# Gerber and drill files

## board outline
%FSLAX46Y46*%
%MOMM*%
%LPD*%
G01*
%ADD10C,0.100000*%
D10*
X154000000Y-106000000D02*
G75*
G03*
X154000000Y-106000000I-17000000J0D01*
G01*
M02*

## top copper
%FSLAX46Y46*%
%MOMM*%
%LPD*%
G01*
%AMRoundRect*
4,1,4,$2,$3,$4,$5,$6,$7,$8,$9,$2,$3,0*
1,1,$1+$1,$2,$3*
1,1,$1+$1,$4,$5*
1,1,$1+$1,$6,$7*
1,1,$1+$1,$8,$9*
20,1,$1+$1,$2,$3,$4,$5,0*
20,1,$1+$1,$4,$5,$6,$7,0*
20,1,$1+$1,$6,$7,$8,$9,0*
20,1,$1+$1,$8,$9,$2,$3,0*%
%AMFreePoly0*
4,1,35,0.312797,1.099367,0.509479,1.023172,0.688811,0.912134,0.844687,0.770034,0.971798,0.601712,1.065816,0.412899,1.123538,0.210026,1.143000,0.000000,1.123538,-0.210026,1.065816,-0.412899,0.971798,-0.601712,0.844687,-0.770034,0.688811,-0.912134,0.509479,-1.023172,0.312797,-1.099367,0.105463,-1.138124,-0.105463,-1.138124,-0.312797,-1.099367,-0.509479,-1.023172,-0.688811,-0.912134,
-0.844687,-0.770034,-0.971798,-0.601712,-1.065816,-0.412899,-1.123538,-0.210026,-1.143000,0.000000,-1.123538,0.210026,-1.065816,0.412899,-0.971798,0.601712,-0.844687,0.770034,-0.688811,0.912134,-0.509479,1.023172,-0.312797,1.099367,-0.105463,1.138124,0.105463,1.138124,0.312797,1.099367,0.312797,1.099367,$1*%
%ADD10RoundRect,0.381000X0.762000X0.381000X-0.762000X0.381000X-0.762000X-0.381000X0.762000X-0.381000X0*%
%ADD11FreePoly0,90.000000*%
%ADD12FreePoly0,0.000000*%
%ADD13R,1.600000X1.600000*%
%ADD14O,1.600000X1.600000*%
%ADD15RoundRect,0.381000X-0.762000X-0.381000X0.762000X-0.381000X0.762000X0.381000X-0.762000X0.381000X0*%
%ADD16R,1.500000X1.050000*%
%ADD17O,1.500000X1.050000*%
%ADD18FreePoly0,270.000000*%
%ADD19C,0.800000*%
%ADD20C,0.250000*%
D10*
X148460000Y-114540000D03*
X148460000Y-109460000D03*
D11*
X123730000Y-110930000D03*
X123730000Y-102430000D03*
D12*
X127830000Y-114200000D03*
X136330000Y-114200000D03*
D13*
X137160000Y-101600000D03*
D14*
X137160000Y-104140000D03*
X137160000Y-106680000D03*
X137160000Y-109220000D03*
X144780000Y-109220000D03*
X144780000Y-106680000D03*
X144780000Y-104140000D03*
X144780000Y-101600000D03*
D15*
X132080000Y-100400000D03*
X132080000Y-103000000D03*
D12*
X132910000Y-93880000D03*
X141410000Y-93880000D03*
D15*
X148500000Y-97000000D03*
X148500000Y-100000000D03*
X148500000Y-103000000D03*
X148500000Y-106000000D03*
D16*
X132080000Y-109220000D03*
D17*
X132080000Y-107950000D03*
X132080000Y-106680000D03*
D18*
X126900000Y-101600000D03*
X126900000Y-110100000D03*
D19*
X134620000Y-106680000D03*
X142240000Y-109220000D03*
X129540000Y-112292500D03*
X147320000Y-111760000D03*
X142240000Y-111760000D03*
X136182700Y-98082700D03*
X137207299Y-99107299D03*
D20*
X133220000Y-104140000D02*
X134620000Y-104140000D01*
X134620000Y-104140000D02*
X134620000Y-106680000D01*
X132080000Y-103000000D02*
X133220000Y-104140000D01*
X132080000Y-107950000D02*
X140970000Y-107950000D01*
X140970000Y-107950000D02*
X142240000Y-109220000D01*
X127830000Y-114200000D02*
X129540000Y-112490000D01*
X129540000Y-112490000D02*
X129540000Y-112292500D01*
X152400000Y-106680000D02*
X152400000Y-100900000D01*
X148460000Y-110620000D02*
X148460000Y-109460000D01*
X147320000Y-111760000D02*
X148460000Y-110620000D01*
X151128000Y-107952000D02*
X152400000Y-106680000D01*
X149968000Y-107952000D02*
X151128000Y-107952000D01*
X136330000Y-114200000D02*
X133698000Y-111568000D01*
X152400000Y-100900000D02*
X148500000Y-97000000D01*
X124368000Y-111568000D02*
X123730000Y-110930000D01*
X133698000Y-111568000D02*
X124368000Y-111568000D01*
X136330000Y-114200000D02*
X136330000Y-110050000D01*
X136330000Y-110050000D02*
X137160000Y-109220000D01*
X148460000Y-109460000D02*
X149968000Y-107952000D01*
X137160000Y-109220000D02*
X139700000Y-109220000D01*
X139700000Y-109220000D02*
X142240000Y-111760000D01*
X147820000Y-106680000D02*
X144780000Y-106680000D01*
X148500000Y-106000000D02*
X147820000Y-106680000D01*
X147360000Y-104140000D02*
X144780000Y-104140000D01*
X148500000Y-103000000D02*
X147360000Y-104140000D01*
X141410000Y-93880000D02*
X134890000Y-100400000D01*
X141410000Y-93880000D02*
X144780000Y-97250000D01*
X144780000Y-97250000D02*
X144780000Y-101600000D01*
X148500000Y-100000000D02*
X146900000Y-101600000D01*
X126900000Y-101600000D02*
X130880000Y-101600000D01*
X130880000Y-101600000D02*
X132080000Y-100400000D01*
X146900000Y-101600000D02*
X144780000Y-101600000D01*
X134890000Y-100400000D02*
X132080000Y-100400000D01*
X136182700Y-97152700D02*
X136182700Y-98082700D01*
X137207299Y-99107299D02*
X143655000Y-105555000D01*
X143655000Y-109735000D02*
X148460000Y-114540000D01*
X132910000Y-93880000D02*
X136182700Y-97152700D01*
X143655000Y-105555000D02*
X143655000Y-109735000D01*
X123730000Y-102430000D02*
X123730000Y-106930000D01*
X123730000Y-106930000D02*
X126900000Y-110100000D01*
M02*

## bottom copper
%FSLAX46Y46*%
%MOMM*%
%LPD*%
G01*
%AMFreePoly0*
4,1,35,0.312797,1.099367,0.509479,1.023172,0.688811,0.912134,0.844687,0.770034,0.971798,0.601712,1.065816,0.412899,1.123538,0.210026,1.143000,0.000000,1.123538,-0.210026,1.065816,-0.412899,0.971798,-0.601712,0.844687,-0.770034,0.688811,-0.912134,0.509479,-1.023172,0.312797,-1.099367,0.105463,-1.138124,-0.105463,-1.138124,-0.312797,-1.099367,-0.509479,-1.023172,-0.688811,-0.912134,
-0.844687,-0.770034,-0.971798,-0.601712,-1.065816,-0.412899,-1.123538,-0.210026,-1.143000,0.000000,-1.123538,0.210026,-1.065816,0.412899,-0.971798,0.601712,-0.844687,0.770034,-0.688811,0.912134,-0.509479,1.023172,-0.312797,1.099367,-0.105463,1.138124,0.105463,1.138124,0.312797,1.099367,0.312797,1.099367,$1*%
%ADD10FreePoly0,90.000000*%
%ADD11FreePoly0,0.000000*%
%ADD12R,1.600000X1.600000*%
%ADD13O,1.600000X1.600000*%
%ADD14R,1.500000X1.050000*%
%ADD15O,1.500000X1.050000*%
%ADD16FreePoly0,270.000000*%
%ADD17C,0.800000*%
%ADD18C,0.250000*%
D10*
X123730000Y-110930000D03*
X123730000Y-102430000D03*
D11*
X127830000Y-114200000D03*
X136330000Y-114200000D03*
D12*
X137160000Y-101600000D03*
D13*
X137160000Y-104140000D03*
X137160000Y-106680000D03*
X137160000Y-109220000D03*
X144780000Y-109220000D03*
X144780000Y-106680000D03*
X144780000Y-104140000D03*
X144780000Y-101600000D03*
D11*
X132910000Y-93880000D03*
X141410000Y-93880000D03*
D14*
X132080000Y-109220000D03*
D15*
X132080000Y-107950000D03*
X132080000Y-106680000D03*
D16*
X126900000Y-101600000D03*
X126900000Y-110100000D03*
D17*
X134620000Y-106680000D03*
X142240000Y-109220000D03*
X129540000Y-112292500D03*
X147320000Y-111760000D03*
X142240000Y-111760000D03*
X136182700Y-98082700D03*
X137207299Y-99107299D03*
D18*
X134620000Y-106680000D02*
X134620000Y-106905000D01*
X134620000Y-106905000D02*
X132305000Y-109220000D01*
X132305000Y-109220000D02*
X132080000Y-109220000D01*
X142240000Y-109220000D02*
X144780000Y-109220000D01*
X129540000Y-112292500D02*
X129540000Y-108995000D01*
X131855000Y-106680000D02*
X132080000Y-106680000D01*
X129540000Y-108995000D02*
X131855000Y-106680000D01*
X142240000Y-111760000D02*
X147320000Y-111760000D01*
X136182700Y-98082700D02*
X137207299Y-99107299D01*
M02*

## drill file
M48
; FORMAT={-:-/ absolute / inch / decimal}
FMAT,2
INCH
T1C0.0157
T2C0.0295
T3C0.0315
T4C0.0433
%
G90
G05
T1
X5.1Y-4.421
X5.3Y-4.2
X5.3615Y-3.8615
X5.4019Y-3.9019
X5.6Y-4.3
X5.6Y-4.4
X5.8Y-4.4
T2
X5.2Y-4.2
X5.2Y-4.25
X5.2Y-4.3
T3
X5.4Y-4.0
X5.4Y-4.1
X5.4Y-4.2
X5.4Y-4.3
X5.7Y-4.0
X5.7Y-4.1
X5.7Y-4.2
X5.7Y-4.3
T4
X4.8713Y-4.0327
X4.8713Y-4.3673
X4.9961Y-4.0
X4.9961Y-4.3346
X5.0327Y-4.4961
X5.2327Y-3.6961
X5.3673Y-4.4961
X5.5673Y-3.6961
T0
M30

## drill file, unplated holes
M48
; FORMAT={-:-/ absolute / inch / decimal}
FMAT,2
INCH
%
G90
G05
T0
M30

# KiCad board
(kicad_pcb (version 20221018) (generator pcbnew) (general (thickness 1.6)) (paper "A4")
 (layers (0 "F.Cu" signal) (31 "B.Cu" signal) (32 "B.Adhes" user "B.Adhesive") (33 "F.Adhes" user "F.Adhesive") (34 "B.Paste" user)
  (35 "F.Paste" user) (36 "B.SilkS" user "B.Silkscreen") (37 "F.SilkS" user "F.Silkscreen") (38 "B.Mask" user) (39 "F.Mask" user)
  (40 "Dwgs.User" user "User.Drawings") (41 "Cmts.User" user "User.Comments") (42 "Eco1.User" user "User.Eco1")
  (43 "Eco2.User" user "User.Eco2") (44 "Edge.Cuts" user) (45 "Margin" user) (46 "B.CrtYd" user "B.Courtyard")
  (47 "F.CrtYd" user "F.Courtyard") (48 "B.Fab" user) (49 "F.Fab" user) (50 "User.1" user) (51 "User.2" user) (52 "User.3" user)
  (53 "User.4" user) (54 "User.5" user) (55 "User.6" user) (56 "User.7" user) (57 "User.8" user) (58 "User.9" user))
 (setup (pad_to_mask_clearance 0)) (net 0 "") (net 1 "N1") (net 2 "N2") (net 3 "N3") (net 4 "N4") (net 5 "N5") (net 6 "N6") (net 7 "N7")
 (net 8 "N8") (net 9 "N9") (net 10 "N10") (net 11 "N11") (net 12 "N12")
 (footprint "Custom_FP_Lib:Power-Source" (layer "F.Cu") (at 151 112 180)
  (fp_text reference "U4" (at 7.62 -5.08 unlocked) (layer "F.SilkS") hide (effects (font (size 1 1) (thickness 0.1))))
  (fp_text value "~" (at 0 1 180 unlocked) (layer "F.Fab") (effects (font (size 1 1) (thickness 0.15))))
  (pad "1" smd roundrect (at 2.54 -2.54 180) (size 2.286 1.524) (layers "F.Cu" "F.Paste" "F.Mask") (roundrect_rratio 0.25) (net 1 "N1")
   (thermal_bridge_angle 45))
  (pad "2" smd roundrect (at 2.54 2.54 180) (size 2.286 1.524) (layers "F.Cu" "F.Paste" "F.Mask") (roundrect_rratio 0.25) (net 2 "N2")
   (thermal_bridge_angle 45)))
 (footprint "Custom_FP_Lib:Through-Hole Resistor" (layer "F.Cu") (at 125 111.25 90)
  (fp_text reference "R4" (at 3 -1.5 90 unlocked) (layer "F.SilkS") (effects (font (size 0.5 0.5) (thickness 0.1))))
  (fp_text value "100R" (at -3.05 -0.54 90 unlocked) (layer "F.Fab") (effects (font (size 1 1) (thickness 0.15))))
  (pad "1" thru_hole custom (at 0.32 -1.27 90) (size 2.286 2.286) (drill 1.1) (layers "*.Cu" "*.Mask") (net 2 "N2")
   (thermal_bridge_angle 45) (options (clearance outline) (anchor circle)) (primitives))
  (pad "2" thru_hole custom (at 8.82 -1.27 90) (size 2.286 2.286) (drill 1.1) (layers "*.Cu" "*.Mask") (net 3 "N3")
   (thermal_bridge_angle 45) (options (clearance outline) (anchor circle)) (primitives)))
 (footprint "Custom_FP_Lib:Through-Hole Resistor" (layer "F.Cu") (at 127.51 115.47)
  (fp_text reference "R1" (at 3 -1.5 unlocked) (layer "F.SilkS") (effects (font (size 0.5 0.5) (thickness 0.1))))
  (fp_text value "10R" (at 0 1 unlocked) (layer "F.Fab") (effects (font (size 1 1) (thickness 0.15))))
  (pad "1" thru_hole custom (at 0.32 -1.27) (size 2.286 2.286) (drill 1.1) (layers "*.Cu" "*.Mask") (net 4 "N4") (thermal_bridge_angle 45)
   (options (clearance outline) (anchor circle)) (primitives))
  (pad "2" thru_hole custom (at 8.82 -1.27) (size 2.286 2.286) (drill 1.1) (layers "*.Cu" "*.Mask") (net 2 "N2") (thermal_bridge_angle 45)
   (options (clearance outline) (anchor circle)) (primitives)))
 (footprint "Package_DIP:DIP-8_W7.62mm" (layer "F.Cu") (at 137.16 101.6)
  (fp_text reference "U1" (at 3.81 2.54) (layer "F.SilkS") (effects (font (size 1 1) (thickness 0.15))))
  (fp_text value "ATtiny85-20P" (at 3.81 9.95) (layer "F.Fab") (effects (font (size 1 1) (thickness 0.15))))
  (pad "1" thru_hole rect (at 0 0) (size 1.6 1.6) (drill 0.8) (layers "*.Cu" "*.Mask") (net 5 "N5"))
  (pad "2" thru_hole oval (at 0 2.54) (size 1.6 1.6) (drill 0.8) (layers "*.Cu" "*.Mask") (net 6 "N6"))
  (pad "3" thru_hole oval (at 0 5.08) (size 1.6 1.6) (drill 0.8) (layers "*.Cu" "*.Mask") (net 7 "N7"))
  (pad "4" thru_hole oval (at 0 7.62) (size 1.6 1.6) (drill 0.8) (layers "*.Cu" "*.Mask") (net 2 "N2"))
  (pad "5" thru_hole oval (at 7.62 7.62) (size 1.6 1.6) (drill 0.8) (layers "*.Cu" "*.Mask") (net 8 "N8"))
  (pad "6" thru_hole oval (at 7.62 5.08) (size 1.6 1.6) (drill 0.8) (layers "*.Cu" "*.Mask") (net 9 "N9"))
  (pad "7" thru_hole oval (at 7.62 2.54) (size 1.6 1.6) (drill 0.8) (layers "*.Cu" "*.Mask") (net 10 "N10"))
  (pad "8" thru_hole oval (at 7.62 0) (size 1.6 1.6) (drill 0.8) (layers "*.Cu" "*.Mask") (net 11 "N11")))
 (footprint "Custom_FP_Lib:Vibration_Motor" (layer "F.Cu") (at 132.08 103)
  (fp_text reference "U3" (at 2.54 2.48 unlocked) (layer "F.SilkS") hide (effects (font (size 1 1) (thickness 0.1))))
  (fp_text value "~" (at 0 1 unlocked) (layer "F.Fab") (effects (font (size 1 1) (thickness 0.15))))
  (pad "1" smd roundrect (at 0 -2.6) (size 2.286 1.524) (layers "F.Cu" "F.Paste" "F.Mask") (roundrect_rratio 0.25) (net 11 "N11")
   (thermal_bridge_angle 45))
  (pad "2" smd roundrect (at 0 0) (size 2.286 1.524) (layers "F.Cu" "F.Paste" "F.Mask") (roundrect_rratio 0.25) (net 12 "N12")
   (thermal_bridge_angle 45)))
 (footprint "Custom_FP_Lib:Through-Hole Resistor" (layer "F.Cu") (at 132.59 95.15)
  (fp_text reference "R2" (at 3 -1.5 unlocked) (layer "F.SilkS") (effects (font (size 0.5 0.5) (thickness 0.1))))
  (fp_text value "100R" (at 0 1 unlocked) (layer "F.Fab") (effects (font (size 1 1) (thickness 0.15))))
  (pad "1" thru_hole custom (at 0.32 -1.27) (size 2.286 2.286) (drill 1.1) (layers "*.Cu" "*.Mask") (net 1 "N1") (thermal_bridge_angle 45)
   (options (clearance outline) (anchor circle)) (primitives))
  (pad "2" thru_hole custom (at 8.82 -1.27) (size 2.286 2.286) (drill 1.1) (layers "*.Cu" "*.Mask") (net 11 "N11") (thermal_bridge_angle 45)
   (options (clearance outline) (anchor circle)) (primitives)))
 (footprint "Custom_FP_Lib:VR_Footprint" (layer "F.Cu") (at 148.5 103)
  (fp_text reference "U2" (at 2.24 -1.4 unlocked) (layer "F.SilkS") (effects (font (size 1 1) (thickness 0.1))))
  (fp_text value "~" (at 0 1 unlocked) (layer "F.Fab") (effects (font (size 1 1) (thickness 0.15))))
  (pad "1" smd roundrect (at 0 -6) (size 2.286 1.524) (layers "F.Cu" "F.Paste" "F.Mask") (roundrect_rratio 0.25) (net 2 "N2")
   (thermal_bridge_angle 45))
  (pad "2" smd roundrect (at 0 -3) (size 2.286 1.524) (layers "F.Cu" "F.Paste" "F.Mask") (roundrect_rratio 0.25) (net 11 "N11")
   (thermal_bridge_angle 45))
  (pad "3" smd roundrect (at 0 0) (size 2.286 1.524) (layers "F.Cu" "F.Paste" "F.Mask") (roundrect_rratio 0.25) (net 10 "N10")
   (thermal_bridge_angle 45))
  (pad "4" smd roundrect (at 0 3) (size 2.286 1.524) (layers "F.Cu" "F.Paste" "F.Mask") (roundrect_rratio 0.25) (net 9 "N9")
   (thermal_bridge_angle 45)))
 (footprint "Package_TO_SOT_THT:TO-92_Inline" (layer "F.Cu") (at 132.08 109.22 90)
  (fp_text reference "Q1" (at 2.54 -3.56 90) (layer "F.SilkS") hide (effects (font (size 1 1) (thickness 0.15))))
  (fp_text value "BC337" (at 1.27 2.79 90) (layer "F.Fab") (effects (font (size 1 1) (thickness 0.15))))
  (pad "1" thru_hole rect (at 0 0 90) (size 1.05 1.5) (drill 0.75) (layers "*.Cu" "*.Mask") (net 12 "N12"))
  (pad "2" thru_hole oval (at 1.27 0 90) (size 1.05 1.5) (drill 0.75) (layers "*.Cu" "*.Mask") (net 8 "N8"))
  (pad "3" thru_hole oval (at 2.54 0 90) (size 1.05 1.5) (drill 0.75) (layers "*.Cu" "*.Mask") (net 4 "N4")))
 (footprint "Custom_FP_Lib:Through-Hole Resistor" (layer "F.Cu") (at 125.63 101.28 -90)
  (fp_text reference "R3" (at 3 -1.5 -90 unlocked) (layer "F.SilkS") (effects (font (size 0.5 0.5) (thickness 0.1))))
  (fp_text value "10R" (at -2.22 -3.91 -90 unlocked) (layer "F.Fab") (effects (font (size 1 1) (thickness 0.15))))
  (pad "1" thru_hole custom (at 0.32 -1.27 270) (size 2.286 2.286) (drill 1.1) (layers "*.Cu" "*.Mask") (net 11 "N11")
   (thermal_bridge_angle 45) (options (clearance outline) (anchor circle)) (primitives))
  (pad "2" thru_hole custom (at 8.82 -1.27 270) (size 2.286 2.286) (drill 1.1) (layers "*.Cu" "*.Mask") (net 3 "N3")
   (thermal_bridge_angle 45) (options (clearance outline) (anchor circle)) (primitives)))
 (gr_circle (center 137 106) (end 154 106) (stroke (width 0.1) (type default)) (fill none) (layer "Edge.Cuts"))
 (segment (start 133.22 104.14) (end 134.62 104.14) (width 0.25) (layer "F.Cu") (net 12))
 (segment (start 134.62 104.14) (end 134.62 106.68) (width 0.25) (layer "F.Cu") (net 12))
 (segment (start 132.08 103) (end 133.22 104.14) (width 0.25) (layer "F.Cu") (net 12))
 (via (at 134.62 106.68) (size 0.8) (drill 0.4) (layers "F.Cu" "B.Cu") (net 12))
 (segment (start 134.62 106.68) (end 134.62 106.905) (width 0.25) (layer "B.Cu") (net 12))
 (segment (start 134.62 106.905) (end 132.305 109.22) (width 0.25) (layer "B.Cu") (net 12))
 (segment (start 132.305 109.22) (end 132.08 109.22) (width 0.25) (layer "B.Cu") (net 12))
 (segment (start 132.08 107.95) (end 140.97 107.95) (width 0.25) (layer "F.Cu") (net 8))
 (segment (start 140.97 107.95) (end 142.24 109.22) (width 0.25) (layer "F.Cu") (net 8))
 (via (at 142.24 109.22) (size 0.8) (drill 0.4) (layers "F.Cu" "B.Cu") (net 8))
 (segment (start 142.24 109.22) (end 144.78 109.22) (width 0.25) (layer "B.Cu") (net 8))
 (segment (start 127.83 114.2) (end 129.54 112.49) (width 0.25) (layer "F.Cu") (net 4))
 (segment (start 129.54 112.49) (end 129.54 112.2925) (width 0.25) (layer "F.Cu") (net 4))
 (via (at 129.54 112.2925) (size 0.8) (drill 0.4) (layers "F.Cu" "B.Cu") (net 4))
 (segment (start 129.54 112.2925) (end 129.54 108.995) (width 0.25) (layer "B.Cu") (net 4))
 (segment (start 131.855 106.68) (end 132.08 106.68) (width 0.25) (layer "B.Cu") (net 4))
 (segment (start 129.54 108.995) (end 131.855 106.68) (width 0.25) (layer "B.Cu") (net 4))
 (segment (start 152.4 106.68) (end 152.4 100.9) (width 0.25) (layer "F.Cu") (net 2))
 (segment (start 148.46 110.62) (end 148.46 109.46) (width 0.25) (layer "F.Cu") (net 2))
 (segment (start 147.32 111.76) (end 148.46 110.62) (width 0.25) (layer "F.Cu") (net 2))
 (segment (start 151.128 107.952) (end 152.4 106.68) (width 0.25) (layer "F.Cu") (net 2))
 (segment (start 149.968 107.952) (end 151.128 107.952) (width 0.25) (layer "F.Cu") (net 2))
 (segment (start 136.33 114.2) (end 133.698 111.568) (width 0.25) (layer "F.Cu") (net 2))
 (segment (start 152.4 100.9) (end 148.5 97) (width 0.25) (layer "F.Cu") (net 2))
 (segment (start 124.368 111.568) (end 123.73 110.93) (width 0.25) (layer "F.Cu") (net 2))
 (segment (start 133.698 111.568) (end 124.368 111.568) (width 0.25) (layer "F.Cu") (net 2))
 (segment (start 136.33 114.2) (end 136.33 110.05) (width 0.25) (layer "F.Cu") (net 2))
 (segment (start 136.33 110.05) (end 137.16 109.22) (width 0.25) (layer "F.Cu") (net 2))
 (segment (start 148.46 109.46) (end 149.968 107.952) (width 0.25) (layer "F.Cu") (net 2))
 (segment (start 137.16 109.22) (end 139.7 109.22) (width 0.25) (layer "F.Cu") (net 2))
 (segment (start 139.7 109.22) (end 142.24 111.76) (width 0.25) (layer "F.Cu") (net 2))
 (via (at 147.32 111.76) (size 0.8) (drill 0.4) (layers "F.Cu" "B.Cu") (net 2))
 (via (at 142.24 111.76) (size 0.8) (drill 0.4) (layers "F.Cu" "B.Cu") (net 2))
 (segment (start 142.24 111.76) (end 147.32 111.76) (width 0.25) (layer "B.Cu") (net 2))
 (segment (start 147.82 106.68) (end 144.78 106.68) (width 0.25) (layer "F.Cu") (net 9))
 (segment (start 148.5 106) (end 147.82 106.68) (width 0.25) (layer "F.Cu") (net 9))
 (segment (start 147.36 104.14) (end 144.78 104.14) (width 0.25) (layer "F.Cu") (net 10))
 (segment (start 148.5 103) (end 147.36 104.14) (width 0.25) (layer "F.Cu") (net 10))
 (segment (start 141.41 93.88) (end 134.89 100.4) (width 0.25) (layer "F.Cu") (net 11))
 (segment (start 141.41 93.88) (end 144.78 97.25) (width 0.25) (layer "F.Cu") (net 11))
 (segment (start 144.78 97.25) (end 144.78 101.6) (width 0.25) (layer "F.Cu") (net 11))
 (segment (start 148.5 100) (end 146.9 101.6) (width 0.25) (layer "F.Cu") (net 11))
 (segment (start 126.9 101.6) (end 130.88 101.6) (width 0.25) (layer "F.Cu") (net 11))
 (segment (start 130.88 101.6) (end 132.08 100.4) (width 0.25) (layer "F.Cu") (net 11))
 (segment (start 146.9 101.6) (end 144.78 101.6) (width 0.25) (layer "F.Cu") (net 11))
 (segment (start 134.89 100.4) (end 132.08 100.4) (width 0.25) (layer "F.Cu") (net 11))
 (segment (start 136.1827 97.1527) (end 136.1827 98.0827) (width 0.25) (layer "F.Cu") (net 1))
 (segment (start 137.207299 99.107299) (end 143.655 105.555) (width 0.25) (layer "F.Cu") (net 1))
 (segment (start 143.655 109.735) (end 148.46 114.54) (width 0.25) (layer "F.Cu") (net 1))
 (segment (start 132.91 93.88) (end 136.1827 97.1527) (width 0.25) (layer "F.Cu") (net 1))
 (segment (start 143.655 105.555) (end 143.655 109.735) (width 0.25) (layer "F.Cu") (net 1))
 (via (at 136.1827 98.0827) (size 0.8) (drill 0.4) (layers "F.Cu" "B.Cu") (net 1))
 (via (at 137.207299 99.107299) (size 0.8) (drill 0.4) (layers "F.Cu" "B.Cu") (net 1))
 (segment (start 136.1827 98.0827) (end 137.207299 99.107299) (width 0.25) (layer "B.Cu") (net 1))
 (segment (start 123.73 102.43) (end 123.73 106.93) (width 0.25) (layer "F.Cu") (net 3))
 (segment (start 123.73 106.93) (end 126.9 110.1) (width 0.25) (layer "F.Cu") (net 3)))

